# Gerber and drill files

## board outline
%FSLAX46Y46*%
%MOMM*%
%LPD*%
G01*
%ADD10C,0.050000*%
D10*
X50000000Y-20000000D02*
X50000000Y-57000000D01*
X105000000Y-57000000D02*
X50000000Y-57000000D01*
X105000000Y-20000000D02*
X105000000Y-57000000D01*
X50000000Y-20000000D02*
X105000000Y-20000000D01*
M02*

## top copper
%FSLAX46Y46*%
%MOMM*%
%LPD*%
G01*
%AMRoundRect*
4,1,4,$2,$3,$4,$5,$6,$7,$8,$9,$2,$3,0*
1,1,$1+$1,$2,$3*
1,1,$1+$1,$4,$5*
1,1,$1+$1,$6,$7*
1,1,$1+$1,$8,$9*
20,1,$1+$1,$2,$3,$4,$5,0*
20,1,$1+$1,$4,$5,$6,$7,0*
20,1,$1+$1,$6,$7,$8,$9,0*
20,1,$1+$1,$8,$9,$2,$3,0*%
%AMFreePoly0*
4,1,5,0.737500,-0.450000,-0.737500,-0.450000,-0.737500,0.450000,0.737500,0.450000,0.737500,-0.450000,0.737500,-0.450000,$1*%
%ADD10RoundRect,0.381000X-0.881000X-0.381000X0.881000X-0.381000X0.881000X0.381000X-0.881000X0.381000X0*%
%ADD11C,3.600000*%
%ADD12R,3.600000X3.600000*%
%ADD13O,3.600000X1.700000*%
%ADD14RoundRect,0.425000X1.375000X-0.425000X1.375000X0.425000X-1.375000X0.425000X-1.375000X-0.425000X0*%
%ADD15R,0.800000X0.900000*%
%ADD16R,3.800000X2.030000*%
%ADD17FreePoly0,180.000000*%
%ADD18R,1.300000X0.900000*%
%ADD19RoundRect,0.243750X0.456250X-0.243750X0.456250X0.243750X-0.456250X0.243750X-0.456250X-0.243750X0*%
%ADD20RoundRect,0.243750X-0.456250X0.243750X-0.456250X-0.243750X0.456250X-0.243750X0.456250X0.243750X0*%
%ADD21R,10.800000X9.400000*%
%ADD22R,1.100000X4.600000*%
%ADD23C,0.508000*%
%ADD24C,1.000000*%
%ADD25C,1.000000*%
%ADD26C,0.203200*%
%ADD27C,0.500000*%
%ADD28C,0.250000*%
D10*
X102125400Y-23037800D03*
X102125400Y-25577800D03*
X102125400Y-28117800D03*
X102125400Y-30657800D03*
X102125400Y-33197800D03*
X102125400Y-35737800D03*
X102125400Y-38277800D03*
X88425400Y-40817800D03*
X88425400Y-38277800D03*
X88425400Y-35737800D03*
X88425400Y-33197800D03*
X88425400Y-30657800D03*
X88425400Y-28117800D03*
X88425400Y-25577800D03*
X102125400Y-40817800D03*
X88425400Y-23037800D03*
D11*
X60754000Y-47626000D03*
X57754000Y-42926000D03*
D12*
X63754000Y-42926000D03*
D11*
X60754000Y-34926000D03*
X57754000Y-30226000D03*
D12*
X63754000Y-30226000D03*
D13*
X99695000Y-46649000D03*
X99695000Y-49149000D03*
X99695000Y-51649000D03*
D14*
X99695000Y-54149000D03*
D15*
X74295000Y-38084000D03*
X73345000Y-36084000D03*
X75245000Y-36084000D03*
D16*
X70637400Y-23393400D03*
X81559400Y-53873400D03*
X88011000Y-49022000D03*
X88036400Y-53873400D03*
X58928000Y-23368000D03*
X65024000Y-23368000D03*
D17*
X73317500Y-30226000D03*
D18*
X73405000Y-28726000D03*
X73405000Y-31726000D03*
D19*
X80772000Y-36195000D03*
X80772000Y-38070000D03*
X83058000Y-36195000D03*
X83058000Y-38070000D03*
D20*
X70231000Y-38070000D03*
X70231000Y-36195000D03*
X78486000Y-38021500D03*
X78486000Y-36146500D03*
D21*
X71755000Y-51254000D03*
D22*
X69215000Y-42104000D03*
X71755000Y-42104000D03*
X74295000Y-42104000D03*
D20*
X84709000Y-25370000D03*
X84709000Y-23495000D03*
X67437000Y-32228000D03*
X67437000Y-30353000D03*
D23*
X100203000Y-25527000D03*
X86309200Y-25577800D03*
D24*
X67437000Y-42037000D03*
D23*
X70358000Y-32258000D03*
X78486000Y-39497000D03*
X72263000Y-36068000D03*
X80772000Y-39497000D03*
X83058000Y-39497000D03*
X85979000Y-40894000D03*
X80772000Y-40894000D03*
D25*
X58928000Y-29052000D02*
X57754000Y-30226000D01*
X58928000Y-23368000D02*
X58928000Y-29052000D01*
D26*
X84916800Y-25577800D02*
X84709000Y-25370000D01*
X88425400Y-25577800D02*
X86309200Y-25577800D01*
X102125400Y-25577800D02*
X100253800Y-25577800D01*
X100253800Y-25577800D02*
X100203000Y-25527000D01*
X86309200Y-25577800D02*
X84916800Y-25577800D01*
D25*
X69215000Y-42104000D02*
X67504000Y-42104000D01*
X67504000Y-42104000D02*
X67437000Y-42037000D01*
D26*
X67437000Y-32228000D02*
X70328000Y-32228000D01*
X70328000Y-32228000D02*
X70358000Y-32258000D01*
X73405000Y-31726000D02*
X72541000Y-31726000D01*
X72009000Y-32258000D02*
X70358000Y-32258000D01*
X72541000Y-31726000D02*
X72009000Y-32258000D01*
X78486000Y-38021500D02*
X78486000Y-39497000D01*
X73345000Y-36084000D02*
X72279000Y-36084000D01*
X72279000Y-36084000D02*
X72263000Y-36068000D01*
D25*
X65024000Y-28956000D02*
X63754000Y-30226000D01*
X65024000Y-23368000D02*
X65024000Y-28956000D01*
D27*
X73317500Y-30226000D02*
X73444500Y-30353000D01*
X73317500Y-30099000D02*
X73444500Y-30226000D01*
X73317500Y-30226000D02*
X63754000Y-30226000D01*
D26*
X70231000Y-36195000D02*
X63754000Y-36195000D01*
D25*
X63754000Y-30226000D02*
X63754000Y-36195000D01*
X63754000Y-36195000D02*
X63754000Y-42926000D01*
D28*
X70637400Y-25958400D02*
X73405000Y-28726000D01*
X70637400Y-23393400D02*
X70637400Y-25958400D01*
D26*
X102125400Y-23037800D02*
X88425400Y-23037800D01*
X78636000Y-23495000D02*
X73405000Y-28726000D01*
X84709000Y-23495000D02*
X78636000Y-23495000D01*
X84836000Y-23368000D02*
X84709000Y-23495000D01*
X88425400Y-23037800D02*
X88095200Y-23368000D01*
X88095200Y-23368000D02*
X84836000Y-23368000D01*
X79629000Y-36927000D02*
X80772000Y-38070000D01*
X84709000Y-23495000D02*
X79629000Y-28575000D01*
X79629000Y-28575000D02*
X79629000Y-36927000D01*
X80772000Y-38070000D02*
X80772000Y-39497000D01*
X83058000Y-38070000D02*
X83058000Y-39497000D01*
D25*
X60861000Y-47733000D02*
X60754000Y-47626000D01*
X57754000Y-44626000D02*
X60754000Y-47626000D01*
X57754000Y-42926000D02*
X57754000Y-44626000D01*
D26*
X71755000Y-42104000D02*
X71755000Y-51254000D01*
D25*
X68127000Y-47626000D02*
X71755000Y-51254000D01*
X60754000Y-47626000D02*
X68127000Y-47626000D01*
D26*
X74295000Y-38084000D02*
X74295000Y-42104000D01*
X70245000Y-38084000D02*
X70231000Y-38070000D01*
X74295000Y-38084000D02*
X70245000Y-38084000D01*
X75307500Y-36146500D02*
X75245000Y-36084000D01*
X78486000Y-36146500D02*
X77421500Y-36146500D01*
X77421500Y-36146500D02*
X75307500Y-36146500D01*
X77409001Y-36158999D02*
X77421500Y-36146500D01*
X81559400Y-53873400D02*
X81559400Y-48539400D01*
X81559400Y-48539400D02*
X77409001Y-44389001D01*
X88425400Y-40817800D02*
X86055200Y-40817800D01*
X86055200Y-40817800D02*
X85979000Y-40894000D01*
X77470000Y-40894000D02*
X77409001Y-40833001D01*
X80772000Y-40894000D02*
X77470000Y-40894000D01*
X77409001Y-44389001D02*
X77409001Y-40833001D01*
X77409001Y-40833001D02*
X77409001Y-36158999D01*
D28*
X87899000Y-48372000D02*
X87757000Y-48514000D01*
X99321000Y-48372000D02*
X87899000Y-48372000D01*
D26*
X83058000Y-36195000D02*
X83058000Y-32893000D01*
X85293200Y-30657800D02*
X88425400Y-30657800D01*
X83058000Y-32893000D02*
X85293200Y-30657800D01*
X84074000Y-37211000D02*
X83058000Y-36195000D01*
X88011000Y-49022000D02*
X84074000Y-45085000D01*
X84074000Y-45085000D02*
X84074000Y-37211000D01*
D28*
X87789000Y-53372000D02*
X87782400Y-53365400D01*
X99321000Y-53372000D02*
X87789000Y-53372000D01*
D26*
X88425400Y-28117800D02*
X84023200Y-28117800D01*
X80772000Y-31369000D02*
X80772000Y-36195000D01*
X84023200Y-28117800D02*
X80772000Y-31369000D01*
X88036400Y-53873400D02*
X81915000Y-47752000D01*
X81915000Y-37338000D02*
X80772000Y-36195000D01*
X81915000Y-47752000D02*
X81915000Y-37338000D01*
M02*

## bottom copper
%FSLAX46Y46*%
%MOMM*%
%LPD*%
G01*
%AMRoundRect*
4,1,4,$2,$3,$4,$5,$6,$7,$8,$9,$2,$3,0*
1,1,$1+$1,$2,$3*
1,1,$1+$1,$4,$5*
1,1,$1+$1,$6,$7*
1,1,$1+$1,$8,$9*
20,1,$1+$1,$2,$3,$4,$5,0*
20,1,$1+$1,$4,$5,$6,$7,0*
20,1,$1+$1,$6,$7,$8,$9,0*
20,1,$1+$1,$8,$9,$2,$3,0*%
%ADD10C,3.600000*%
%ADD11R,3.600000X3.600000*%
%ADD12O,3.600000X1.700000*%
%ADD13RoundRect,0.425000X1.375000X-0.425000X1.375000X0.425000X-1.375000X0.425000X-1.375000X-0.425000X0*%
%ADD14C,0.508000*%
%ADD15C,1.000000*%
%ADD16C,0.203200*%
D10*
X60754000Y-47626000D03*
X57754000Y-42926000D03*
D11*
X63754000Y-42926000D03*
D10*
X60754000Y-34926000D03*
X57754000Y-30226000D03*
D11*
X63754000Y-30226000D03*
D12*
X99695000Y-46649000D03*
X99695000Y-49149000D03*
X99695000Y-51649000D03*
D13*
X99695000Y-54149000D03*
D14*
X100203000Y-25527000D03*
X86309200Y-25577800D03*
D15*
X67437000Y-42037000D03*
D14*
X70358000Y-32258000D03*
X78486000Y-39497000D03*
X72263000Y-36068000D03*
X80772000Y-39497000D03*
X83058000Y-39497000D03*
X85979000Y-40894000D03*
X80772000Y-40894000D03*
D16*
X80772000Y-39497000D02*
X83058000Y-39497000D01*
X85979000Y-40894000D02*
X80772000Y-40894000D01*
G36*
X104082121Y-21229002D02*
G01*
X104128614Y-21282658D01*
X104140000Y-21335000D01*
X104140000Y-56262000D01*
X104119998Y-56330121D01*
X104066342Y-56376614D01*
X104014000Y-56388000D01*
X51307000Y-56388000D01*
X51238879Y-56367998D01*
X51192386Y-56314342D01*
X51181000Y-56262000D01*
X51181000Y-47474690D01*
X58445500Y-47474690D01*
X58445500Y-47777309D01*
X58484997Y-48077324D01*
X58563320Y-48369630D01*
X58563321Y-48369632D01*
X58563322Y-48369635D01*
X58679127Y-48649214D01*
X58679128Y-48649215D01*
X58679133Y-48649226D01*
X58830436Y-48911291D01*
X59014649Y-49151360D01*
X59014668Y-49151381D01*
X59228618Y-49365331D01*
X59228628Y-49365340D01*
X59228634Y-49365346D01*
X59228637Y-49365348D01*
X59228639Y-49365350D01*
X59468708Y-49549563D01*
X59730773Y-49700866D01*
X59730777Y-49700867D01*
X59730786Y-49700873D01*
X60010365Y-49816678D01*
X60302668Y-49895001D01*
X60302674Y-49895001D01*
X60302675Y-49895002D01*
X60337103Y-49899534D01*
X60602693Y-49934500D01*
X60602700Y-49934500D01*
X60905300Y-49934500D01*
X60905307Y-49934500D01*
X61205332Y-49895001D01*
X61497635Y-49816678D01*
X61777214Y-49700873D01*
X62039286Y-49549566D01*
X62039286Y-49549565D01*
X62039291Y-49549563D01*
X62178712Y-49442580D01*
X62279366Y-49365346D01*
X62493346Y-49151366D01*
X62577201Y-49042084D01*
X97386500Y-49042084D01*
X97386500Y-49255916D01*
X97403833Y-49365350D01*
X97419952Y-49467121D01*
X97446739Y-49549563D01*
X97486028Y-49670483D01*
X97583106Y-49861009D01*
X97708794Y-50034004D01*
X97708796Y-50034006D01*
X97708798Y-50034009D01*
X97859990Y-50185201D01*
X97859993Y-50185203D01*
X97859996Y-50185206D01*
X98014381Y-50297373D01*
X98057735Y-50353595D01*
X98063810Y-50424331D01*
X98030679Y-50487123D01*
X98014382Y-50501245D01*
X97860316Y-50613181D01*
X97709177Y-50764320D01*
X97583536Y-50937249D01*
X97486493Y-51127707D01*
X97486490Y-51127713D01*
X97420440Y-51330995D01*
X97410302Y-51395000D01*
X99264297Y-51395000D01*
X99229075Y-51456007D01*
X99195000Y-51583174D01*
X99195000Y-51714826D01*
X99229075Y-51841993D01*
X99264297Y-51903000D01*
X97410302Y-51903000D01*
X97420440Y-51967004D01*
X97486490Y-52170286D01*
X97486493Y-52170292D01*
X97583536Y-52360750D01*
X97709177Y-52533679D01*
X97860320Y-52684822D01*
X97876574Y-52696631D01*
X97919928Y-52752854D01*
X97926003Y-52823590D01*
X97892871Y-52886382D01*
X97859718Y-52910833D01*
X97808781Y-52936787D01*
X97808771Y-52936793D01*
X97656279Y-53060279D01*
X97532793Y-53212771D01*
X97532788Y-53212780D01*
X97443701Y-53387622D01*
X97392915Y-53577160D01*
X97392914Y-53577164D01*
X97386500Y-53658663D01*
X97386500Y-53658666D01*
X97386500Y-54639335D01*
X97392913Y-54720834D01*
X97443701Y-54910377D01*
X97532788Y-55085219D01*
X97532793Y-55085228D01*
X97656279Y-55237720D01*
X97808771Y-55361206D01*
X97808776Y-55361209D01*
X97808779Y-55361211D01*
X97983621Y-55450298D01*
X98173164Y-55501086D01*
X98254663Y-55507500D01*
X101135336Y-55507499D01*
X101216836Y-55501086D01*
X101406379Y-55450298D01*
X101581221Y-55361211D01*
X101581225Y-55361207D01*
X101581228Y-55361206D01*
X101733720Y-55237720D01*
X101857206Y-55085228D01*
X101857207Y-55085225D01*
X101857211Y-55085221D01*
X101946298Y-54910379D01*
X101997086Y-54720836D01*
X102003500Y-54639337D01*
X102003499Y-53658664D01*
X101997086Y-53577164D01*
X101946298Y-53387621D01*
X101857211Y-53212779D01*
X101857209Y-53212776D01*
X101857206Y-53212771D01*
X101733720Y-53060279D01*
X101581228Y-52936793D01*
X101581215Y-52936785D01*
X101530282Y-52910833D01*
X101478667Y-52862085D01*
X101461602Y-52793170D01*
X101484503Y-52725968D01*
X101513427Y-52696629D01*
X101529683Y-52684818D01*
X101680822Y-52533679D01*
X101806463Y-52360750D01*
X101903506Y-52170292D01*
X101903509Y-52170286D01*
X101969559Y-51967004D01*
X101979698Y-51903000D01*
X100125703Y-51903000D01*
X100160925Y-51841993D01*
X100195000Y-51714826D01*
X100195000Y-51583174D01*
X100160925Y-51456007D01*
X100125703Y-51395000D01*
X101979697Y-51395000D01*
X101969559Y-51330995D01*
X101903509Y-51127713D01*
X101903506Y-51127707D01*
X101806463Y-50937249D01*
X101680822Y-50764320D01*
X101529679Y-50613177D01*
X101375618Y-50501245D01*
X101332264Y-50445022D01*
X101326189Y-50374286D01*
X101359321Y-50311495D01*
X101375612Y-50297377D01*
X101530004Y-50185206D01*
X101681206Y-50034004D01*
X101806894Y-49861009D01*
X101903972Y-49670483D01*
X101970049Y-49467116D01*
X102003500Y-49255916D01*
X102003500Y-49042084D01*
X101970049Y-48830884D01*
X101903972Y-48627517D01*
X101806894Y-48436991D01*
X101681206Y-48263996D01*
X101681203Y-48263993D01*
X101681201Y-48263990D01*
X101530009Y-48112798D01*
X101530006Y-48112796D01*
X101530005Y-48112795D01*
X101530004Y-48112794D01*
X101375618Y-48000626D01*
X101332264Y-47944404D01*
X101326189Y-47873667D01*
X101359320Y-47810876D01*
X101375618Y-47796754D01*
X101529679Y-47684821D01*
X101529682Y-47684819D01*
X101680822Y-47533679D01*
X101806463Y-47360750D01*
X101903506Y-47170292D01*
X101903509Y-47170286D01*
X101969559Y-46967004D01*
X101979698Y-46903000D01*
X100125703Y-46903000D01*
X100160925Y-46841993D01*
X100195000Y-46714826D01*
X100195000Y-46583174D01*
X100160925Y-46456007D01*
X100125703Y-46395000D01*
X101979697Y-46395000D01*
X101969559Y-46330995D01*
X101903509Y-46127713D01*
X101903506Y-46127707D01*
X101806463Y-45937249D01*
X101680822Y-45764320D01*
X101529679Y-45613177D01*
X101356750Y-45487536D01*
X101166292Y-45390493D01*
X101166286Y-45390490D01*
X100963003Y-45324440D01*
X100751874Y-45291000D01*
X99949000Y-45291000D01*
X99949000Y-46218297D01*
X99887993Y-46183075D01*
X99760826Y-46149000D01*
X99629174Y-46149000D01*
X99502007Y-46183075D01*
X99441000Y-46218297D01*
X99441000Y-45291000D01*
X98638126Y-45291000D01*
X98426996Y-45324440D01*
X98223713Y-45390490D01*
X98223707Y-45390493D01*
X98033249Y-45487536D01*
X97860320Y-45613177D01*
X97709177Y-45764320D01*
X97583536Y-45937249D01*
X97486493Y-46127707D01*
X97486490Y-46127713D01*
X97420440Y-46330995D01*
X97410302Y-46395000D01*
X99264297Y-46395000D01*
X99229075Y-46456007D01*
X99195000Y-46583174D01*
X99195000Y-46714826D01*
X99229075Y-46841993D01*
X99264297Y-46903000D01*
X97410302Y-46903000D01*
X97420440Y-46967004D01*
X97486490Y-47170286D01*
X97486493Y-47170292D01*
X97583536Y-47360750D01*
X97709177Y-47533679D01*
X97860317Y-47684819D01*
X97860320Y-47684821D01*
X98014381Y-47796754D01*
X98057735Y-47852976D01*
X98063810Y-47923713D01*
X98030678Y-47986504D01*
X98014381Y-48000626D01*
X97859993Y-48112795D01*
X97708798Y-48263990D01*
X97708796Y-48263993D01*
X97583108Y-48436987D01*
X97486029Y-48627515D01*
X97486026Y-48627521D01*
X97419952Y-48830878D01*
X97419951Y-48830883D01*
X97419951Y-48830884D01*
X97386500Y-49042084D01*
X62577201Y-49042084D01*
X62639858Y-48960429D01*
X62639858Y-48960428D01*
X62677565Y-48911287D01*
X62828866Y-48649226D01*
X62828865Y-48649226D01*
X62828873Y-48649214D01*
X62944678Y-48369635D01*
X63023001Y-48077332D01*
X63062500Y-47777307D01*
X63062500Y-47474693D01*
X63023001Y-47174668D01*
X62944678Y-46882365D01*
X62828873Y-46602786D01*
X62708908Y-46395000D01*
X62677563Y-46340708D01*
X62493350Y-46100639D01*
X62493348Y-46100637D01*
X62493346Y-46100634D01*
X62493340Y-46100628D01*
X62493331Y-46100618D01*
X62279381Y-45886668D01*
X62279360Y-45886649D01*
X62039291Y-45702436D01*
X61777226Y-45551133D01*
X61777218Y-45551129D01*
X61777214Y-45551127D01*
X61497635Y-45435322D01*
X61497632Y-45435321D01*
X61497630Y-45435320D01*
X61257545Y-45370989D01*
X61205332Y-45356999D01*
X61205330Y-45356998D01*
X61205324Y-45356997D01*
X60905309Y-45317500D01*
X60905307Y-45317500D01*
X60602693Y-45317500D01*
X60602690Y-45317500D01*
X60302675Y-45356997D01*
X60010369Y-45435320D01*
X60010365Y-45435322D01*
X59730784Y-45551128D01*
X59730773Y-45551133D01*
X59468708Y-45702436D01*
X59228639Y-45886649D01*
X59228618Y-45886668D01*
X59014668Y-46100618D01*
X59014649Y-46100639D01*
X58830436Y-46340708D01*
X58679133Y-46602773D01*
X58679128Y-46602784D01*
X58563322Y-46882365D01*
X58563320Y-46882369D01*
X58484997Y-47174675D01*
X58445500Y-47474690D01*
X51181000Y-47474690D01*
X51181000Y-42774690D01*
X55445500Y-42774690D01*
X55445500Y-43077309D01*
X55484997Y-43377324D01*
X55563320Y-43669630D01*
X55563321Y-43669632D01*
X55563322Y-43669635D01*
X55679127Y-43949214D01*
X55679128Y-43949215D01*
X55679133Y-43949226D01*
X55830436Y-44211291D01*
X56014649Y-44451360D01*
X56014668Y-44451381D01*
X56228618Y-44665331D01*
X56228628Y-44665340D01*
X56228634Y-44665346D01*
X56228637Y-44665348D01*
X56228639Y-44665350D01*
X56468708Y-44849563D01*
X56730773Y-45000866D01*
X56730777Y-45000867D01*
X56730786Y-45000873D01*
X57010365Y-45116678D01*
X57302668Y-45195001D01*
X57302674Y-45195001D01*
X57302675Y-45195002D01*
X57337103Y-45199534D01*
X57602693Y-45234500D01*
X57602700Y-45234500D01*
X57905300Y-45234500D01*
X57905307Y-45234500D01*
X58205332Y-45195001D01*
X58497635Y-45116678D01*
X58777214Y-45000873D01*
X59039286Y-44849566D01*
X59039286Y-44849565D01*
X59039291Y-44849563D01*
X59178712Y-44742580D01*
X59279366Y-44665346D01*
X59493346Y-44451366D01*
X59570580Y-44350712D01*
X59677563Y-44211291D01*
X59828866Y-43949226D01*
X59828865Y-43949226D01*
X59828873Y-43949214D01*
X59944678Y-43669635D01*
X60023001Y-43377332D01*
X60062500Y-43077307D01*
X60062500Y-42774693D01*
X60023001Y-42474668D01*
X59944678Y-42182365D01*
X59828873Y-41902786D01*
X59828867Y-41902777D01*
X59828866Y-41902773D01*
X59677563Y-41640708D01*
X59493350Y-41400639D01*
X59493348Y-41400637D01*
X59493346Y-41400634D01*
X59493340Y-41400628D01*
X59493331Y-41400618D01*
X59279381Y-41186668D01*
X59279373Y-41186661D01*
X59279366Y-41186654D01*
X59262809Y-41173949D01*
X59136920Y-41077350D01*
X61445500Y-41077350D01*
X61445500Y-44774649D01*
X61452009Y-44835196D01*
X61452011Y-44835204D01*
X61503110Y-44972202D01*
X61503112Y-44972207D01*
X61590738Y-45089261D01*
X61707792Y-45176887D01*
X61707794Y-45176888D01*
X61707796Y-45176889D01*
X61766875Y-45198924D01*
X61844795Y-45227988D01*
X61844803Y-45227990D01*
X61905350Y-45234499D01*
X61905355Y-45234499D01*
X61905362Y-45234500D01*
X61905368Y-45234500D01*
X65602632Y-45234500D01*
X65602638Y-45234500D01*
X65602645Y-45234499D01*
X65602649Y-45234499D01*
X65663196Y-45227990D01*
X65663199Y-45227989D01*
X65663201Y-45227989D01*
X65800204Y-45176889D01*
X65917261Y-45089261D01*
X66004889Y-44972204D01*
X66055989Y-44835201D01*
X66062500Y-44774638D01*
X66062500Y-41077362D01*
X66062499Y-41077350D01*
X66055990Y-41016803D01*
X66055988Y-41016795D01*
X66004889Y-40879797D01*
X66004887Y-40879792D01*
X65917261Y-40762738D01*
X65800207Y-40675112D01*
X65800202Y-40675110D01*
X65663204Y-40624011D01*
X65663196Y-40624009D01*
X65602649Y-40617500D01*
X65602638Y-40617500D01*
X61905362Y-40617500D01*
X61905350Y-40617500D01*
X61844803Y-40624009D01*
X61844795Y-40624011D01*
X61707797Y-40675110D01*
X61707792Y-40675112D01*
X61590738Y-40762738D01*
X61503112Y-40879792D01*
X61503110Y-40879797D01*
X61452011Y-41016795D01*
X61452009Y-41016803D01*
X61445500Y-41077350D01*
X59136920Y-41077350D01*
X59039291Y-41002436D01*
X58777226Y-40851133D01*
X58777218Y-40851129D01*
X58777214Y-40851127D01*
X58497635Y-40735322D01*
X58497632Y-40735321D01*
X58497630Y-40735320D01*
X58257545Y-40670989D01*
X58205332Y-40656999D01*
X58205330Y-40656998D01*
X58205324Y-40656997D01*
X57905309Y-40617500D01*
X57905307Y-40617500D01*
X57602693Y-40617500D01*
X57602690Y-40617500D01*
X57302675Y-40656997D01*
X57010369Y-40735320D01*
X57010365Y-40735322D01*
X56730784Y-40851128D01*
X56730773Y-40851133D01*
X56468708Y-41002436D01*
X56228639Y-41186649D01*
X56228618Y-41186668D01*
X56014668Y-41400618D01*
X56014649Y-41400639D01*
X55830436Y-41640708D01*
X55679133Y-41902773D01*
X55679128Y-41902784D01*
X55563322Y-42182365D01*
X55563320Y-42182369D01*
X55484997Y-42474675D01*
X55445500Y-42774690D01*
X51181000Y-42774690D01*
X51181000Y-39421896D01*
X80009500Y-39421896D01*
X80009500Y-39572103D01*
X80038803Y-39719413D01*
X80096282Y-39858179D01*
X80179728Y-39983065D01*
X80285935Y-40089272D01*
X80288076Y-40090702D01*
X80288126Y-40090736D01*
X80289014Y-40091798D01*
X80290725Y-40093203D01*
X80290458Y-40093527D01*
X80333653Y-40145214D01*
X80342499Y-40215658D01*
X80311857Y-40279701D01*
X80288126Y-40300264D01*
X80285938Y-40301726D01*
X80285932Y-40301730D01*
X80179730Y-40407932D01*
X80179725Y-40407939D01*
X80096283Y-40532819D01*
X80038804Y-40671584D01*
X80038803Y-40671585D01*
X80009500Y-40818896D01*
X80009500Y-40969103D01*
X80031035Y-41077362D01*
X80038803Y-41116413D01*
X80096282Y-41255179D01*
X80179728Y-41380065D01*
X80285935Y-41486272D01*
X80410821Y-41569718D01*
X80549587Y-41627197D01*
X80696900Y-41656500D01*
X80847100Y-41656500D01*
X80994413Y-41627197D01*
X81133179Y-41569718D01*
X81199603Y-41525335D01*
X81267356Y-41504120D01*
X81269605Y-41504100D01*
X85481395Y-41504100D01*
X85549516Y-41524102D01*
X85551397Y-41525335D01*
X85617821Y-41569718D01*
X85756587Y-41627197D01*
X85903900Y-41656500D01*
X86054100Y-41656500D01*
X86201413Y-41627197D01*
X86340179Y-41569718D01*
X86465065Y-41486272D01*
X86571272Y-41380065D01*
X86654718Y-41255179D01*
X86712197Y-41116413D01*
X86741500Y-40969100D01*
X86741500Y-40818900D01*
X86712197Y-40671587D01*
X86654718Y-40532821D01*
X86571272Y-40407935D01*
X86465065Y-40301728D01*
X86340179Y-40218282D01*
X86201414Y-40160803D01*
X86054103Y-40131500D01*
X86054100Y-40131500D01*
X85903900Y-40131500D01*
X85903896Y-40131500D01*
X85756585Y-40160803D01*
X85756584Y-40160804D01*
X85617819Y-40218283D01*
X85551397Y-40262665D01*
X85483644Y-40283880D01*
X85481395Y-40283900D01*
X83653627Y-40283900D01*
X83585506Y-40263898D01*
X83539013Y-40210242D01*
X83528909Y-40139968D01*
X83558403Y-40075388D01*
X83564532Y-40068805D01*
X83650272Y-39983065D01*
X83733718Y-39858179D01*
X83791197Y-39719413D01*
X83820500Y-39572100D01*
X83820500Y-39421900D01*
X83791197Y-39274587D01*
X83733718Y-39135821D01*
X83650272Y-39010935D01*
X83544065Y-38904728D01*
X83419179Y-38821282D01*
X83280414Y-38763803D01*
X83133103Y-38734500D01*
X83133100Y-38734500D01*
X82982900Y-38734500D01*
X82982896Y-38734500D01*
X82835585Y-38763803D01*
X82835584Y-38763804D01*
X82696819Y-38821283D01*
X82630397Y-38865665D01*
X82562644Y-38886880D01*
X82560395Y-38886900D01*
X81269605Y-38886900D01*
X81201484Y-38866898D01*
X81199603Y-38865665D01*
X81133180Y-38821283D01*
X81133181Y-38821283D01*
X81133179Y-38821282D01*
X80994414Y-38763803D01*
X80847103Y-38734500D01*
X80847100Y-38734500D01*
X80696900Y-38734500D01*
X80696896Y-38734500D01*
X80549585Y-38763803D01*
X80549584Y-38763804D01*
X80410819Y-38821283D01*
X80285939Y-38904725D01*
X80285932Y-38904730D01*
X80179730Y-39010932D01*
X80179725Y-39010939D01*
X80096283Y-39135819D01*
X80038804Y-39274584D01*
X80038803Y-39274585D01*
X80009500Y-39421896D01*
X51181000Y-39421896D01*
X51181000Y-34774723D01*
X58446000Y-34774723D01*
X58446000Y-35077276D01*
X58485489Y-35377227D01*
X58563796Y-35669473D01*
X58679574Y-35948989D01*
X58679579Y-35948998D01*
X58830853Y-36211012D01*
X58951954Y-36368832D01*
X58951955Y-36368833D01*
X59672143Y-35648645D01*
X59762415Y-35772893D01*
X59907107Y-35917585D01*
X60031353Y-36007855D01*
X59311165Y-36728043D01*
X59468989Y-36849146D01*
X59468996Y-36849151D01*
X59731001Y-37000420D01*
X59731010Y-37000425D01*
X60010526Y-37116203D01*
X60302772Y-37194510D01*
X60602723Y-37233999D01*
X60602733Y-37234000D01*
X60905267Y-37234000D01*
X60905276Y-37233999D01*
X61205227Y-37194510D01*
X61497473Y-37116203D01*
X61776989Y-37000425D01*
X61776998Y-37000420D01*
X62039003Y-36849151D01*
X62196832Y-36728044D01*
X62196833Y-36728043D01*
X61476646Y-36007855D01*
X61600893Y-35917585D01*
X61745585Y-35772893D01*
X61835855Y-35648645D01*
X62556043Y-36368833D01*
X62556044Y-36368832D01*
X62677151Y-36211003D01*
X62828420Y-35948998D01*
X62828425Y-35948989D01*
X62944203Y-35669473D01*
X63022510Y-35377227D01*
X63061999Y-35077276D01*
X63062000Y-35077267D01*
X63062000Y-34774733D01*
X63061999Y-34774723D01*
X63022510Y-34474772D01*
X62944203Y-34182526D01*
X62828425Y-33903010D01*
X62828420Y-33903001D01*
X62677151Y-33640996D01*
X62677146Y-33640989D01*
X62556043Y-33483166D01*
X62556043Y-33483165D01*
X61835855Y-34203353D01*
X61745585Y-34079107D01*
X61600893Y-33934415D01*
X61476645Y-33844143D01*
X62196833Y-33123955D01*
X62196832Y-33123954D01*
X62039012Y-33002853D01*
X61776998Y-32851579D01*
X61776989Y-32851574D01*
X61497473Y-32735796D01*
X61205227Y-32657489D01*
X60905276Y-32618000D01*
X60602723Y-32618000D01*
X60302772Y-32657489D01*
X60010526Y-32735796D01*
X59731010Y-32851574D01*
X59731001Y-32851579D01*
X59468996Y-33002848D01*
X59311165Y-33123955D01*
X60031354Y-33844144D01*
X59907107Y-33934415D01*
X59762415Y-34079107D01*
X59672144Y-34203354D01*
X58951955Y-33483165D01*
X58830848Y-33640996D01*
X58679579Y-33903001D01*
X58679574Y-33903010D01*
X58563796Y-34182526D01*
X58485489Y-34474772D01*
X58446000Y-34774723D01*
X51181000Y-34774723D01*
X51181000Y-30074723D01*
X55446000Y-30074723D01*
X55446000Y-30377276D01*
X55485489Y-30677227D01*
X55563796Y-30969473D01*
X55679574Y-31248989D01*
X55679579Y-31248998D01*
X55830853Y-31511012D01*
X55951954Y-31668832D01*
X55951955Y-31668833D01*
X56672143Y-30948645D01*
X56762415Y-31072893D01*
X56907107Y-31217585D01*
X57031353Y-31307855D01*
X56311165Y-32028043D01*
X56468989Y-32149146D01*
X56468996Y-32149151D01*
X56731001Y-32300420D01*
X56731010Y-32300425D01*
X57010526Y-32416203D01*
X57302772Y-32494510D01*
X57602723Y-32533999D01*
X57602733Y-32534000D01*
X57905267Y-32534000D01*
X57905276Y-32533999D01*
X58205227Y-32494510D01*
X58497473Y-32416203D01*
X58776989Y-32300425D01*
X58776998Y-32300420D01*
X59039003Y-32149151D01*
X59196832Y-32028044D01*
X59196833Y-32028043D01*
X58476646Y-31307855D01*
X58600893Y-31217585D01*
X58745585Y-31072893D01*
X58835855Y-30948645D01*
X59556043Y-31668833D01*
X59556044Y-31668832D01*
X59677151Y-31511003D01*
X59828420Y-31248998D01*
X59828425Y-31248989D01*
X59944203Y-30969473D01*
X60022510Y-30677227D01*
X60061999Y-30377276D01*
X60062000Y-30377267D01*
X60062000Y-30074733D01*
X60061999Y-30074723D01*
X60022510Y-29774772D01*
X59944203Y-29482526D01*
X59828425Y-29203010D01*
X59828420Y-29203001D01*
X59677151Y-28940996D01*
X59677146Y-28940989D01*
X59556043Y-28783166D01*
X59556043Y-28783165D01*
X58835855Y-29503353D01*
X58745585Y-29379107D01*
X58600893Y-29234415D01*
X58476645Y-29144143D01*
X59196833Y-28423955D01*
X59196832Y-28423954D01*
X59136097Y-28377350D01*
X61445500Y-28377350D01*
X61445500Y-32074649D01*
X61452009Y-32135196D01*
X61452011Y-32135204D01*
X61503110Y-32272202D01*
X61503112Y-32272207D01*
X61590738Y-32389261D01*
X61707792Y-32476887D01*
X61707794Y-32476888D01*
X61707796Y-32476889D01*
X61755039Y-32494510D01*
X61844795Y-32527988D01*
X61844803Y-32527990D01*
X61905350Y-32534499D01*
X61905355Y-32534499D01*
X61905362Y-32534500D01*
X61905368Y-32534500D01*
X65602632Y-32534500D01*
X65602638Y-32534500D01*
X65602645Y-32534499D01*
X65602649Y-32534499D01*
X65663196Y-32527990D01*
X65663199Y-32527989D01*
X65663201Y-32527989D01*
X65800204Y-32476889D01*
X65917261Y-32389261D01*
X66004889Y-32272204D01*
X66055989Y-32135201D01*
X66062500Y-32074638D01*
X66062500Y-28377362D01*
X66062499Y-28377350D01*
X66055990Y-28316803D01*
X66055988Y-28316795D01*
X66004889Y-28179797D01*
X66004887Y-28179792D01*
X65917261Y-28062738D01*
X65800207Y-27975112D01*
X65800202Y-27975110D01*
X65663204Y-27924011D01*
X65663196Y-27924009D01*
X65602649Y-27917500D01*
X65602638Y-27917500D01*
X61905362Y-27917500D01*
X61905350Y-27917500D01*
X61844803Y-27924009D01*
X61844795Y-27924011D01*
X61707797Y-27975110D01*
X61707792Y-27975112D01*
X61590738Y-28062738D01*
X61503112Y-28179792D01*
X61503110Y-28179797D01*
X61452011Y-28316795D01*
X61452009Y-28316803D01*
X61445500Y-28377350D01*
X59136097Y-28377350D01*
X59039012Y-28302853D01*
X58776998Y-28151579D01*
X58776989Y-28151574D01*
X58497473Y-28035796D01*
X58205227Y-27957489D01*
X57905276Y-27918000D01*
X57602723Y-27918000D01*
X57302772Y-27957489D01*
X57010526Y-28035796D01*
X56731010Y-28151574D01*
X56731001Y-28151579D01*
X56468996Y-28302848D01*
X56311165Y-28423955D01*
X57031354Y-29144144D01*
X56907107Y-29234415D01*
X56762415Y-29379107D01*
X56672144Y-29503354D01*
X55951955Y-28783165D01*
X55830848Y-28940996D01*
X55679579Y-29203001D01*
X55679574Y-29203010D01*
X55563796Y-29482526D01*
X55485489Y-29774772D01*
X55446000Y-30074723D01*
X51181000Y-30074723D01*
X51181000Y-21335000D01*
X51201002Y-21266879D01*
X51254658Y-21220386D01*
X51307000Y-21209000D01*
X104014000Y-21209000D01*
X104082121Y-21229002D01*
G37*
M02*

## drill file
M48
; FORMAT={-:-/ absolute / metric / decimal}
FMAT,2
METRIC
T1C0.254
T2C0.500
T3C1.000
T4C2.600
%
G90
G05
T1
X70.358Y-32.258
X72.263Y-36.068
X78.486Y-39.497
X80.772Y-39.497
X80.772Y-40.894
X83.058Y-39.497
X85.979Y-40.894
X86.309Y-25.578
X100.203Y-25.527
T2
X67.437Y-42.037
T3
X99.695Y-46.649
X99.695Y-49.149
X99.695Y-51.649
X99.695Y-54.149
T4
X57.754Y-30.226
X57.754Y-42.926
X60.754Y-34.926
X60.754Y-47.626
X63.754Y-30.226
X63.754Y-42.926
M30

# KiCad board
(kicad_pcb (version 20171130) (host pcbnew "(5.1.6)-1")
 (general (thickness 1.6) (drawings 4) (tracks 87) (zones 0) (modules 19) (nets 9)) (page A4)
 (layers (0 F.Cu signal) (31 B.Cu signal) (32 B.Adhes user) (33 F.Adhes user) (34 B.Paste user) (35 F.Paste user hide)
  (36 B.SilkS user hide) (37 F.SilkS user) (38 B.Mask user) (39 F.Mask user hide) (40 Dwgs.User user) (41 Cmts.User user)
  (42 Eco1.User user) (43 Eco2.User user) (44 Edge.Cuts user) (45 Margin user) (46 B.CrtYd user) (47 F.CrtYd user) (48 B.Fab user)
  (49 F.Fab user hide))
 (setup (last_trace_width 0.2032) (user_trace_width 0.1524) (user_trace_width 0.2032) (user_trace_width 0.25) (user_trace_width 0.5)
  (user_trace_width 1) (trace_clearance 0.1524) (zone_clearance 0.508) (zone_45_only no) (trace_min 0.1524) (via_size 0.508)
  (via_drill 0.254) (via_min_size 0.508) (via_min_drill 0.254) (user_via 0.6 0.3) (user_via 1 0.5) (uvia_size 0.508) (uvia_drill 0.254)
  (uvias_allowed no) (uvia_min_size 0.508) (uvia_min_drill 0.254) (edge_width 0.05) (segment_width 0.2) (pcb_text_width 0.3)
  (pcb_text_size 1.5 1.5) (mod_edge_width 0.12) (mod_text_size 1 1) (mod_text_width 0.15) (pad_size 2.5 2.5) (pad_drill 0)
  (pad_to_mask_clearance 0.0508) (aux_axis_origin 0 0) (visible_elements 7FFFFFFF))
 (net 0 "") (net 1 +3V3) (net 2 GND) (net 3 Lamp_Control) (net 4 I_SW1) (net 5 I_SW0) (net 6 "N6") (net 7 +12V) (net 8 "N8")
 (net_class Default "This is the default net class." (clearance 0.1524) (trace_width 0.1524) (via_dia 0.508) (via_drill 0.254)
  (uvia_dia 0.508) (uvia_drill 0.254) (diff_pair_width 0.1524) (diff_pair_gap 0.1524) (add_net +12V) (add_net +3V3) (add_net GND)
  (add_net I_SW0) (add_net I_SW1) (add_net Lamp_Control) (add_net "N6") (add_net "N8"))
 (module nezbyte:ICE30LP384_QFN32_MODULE (layer F.Cu) (at 95.25 31.75)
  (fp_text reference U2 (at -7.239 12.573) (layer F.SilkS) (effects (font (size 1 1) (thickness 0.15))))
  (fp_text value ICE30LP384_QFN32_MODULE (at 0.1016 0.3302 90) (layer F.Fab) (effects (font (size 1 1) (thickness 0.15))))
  (pad 16 smd roundrect (at 6.8754 -8.7122) (size 2.524 1.524) (layers F.Cu F.Paste F.Mask) (roundrect_rratio 0.25) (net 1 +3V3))
  (pad 15 smd roundrect (at 6.8754 -6.1722) (size 2.524 1.524) (layers F.Cu F.Paste F.Mask) (roundrect_rratio 0.25) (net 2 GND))
  (pad 14 smd roundrect (at 6.8754 -3.6322) (size 2.524 1.524) (layers F.Cu F.Paste F.Mask) (roundrect_rratio 0.25))
  (pad 13 smd roundrect (at 6.8754 -1.0922) (size 2.524 1.524) (layers F.Cu F.Paste F.Mask) (roundrect_rratio 0.25))
  (pad 12 smd roundrect (at 6.8754 1.4478) (size 2.524 1.524) (layers F.Cu F.Paste F.Mask) (roundrect_rratio 0.25))
  (pad 11 smd roundrect (at 6.8754 3.9878) (size 2.524 1.524) (layers F.Cu F.Paste F.Mask) (roundrect_rratio 0.25))
  (pad 10 smd roundrect (at 6.8754 6.5278) (size 2.524 1.524) (layers F.Cu F.Paste F.Mask) (roundrect_rratio 0.25))
  (pad 8 smd roundrect (at -6.8246 9.0678) (size 2.524 1.524) (layers F.Cu F.Paste F.Mask) (roundrect_rratio 0.25) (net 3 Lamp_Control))
  (pad 7 smd roundrect (at -6.8246 6.5278) (size 2.524 1.524) (layers F.Cu F.Paste F.Mask) (roundrect_rratio 0.25))
  (pad 6 smd roundrect (at -6.8246 3.9878) (size 2.524 1.524) (layers F.Cu F.Paste F.Mask) (roundrect_rratio 0.25))
  (pad 5 smd roundrect (at -6.8246 1.4478) (size 2.524 1.524) (layers F.Cu F.Paste F.Mask) (roundrect_rratio 0.25))
  (pad 4 smd roundrect (at -6.8246 -1.0922) (size 2.524 1.524) (layers F.Cu F.Paste F.Mask) (roundrect_rratio 0.25) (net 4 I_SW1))
  (pad 3 smd roundrect (at -6.8246 -3.6322) (size 2.524 1.524) (layers F.Cu F.Paste F.Mask) (roundrect_rratio 0.25) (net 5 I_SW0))
  (pad 2 smd roundrect (at -6.8246 -6.1722) (size 2.524 1.524) (layers F.Cu F.Paste F.Mask) (roundrect_rratio 0.25) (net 2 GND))
  (pad 9 smd roundrect (at 6.8754 9.0678) (size 2.524 1.524) (layers F.Cu F.Paste F.Mask) (roundrect_rratio 0.25))
  (pad 1 smd roundrect (at -6.8246 -8.7122) (size 2.524 1.524) (layers F.Cu F.Paste F.Mask) (roundrect_rratio 0.25) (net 1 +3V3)))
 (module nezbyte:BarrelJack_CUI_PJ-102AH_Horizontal (layer F.Cu) (at 63.754 42.926 270)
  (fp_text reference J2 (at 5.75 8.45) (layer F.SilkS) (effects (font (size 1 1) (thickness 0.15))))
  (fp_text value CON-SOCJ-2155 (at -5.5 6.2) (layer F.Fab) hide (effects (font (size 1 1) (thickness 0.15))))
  (pad 3 thru_hole circle (at 4.7 3 270) (size 3.6 3.6) (drill 2.6) (layers *.Cu *.Mask) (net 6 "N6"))
  (pad 2 thru_hole circle (at 0 6 270) (size 3.6 3.6) (drill 2.6) (layers *.Cu *.Mask) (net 6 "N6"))
  (pad 1 thru_hole rect (at 0 0 270) (size 3.6 3.6) (drill 2.6) (layers *.Cu *.Mask) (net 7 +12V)))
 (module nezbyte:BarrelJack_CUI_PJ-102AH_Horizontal (layer F.Cu) (at 63.754 30.226 270)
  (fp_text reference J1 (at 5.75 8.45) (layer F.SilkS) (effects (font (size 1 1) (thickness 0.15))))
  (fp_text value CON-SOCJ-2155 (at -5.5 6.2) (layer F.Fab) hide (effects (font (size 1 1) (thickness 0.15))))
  (pad 3 thru_hole circle (at 4.7 3 270) (size 3.6 3.6) (drill 2.6) (layers *.Cu *.Mask) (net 2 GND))
  (pad 2 thru_hole circle (at 0 6 270) (size 3.6 3.6) (drill 2.6) (layers *.Cu *.Mask) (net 2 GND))
  (pad 1 thru_hole rect (at 0 0 270) (size 3.6 3.6) (drill 2.6) (layers *.Cu *.Mask) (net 7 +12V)))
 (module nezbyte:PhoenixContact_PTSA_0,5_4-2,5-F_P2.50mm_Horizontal (layer F.Cu) (at 92.195 56.149 90)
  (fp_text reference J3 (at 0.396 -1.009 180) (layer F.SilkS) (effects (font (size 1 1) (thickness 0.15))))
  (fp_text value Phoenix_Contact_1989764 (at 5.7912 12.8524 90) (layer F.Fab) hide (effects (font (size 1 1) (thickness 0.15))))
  (pad 4 thru_hole oval (at 9.5 7.5 90) (size 1.7 3.6) (drill 1) (layers *.Cu *.Mask) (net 2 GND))
  (pad 3 thru_hole oval (at 7 7.5 90) (size 1.7 3.6) (drill 1) (layers *.Cu *.Mask) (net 4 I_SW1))
  (pad 2 thru_hole oval (at 4.5 7.5 90) (size 1.7 3.6) (drill 1) (layers *.Cu *.Mask) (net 2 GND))
  (pad 1 thru_hole roundrect (at 2 7.5 90) (size 1.7 3.6) (drill 1) (layers *.Cu *.Mask) (roundrect_rratio 0.25) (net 5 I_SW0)))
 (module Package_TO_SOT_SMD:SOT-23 (layer F.Cu) (at 74.295 37.084 270)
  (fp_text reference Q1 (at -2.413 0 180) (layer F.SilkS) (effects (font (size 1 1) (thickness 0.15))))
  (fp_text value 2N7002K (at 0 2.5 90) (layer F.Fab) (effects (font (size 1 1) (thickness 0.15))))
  (pad 3 smd rect (at 1 0 270) (size 0.9 0.8) (layers F.Cu F.Paste F.Mask) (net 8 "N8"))
  (pad 2 smd rect (at -1 0.95 270) (size 0.9 0.8) (layers F.Cu F.Paste F.Mask) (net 2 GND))
  (pad 1 smd rect (at -1 -0.95 270) (size 0.9 0.8) (layers F.Cu F.Paste F.Mask) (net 3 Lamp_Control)))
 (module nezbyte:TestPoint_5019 (layer F.Cu) (at 70.612 23.368)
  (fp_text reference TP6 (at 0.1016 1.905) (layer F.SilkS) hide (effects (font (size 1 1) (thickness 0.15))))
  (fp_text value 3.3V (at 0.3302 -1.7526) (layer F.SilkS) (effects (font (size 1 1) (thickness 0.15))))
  (pad 1 smd rect (at 0.0254 0.0254) (size 3.8 2.03) (layers F.Cu F.Paste F.Mask) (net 1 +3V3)))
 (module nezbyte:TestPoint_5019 (layer F.Cu) (at 81.534 53.848)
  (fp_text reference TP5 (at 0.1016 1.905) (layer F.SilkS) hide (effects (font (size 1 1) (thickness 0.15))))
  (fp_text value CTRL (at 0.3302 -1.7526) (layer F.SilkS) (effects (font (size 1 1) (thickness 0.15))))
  (pad 1 smd rect (at 0.0254 0.0254) (size 3.8 2.03) (layers F.Cu F.Paste F.Mask) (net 3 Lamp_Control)))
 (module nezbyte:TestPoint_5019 (layer F.Cu) (at 87.9856 48.9966)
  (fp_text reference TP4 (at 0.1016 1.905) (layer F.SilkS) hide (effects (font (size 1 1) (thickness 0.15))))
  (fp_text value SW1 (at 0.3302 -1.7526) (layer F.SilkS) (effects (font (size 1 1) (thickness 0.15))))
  (pad 1 smd rect (at 0.0254 0.0254) (size 3.8 2.03) (layers F.Cu F.Paste F.Mask) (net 4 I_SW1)))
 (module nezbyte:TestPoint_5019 (layer F.Cu) (at 88.011 53.848)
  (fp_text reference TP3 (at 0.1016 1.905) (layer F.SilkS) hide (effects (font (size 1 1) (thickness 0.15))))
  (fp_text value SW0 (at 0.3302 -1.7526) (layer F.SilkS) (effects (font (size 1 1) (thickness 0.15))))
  (pad 1 smd rect (at 0.0254 0.0254) (size 3.8 2.03) (layers F.Cu F.Paste F.Mask) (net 5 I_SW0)))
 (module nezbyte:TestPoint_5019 (layer F.Cu) (at 58.9026 23.3426)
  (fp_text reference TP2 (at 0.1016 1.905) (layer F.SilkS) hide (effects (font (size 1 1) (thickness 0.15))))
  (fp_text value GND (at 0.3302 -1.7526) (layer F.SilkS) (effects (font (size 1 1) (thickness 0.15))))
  (pad 1 smd rect (at 0.0254 0.0254) (size 3.8 2.03) (layers F.Cu F.Paste F.Mask) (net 2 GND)))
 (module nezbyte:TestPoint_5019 (layer F.Cu) (at 64.9986 23.3426)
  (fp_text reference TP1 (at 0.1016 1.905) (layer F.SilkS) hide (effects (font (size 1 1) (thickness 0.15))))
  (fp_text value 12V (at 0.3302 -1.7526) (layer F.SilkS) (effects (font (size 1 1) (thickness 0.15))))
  (pad 1 smd rect (at 0.0254 0.0254) (size 3.8 2.03) (layers F.Cu F.Paste F.Mask) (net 7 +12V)))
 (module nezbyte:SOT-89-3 (layer F.Cu) (at 71.755 30.226 180)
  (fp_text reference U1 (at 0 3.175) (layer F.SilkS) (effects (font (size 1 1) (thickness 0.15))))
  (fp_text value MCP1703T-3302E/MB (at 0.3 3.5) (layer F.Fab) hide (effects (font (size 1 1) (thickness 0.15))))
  (pad 2 smd custom (at -1.5625 0 180) (size 1.475 0.9) (layers F.Cu F.Paste F.Mask) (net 7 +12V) (zone_connect 2)
   (options (clearance outline) (anchor rect)) (primitives))
  (pad 3 smd rect (at -1.65 1.5 180) (size 1.3 0.9) (layers F.Cu F.Paste F.Mask) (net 1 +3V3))
  (pad 1 smd rect (at -1.65 -1.5 180) (size 1.3 0.9) (layers F.Cu F.Paste F.Mask) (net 2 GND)))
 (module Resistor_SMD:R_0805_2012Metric (layer F.Cu) (at 80.772 37.1325 90)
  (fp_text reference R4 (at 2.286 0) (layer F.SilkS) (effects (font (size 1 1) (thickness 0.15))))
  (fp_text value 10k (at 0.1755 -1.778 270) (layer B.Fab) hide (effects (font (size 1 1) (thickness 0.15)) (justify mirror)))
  (pad 2 smd roundrect (at 0.9375 0 90) (size 0.975 1.4) (layers F.Cu F.Paste F.Mask) (roundrect_rratio 0.25) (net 5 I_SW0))
  (pad 1 smd roundrect (at -0.9375 0 90) (size 0.975 1.4) (layers F.Cu F.Paste F.Mask) (roundrect_rratio 0.25) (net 1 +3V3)))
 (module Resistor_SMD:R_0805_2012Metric (layer F.Cu) (at 83.058 37.1325 90)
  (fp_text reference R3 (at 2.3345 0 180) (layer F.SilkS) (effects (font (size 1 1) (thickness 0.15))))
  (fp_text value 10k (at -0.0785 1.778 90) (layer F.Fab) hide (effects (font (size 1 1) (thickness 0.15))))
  (pad 2 smd roundrect (at 0.9375 0 90) (size 0.975 1.4) (layers F.Cu F.Paste F.Mask) (roundrect_rratio 0.25) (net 4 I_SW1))
  (pad 1 smd roundrect (at -0.9375 0 90) (size 0.975 1.4) (layers F.Cu F.Paste F.Mask) (roundrect_rratio 0.25) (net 1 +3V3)))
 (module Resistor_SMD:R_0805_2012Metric (layer F.Cu) (at 70.231 37.1325 270)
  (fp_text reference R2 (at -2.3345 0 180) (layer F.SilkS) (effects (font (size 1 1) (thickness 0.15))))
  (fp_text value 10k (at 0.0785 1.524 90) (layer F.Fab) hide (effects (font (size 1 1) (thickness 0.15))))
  (pad 2 smd roundrect (at 0.9375 0 270) (size 0.975 1.4) (layers F.Cu F.Paste F.Mask) (roundrect_rratio 0.25) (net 8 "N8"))
  (pad 1 smd roundrect (at -0.9375 0 270) (size 0.975 1.4) (layers F.Cu F.Paste F.Mask) (roundrect_rratio 0.25) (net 7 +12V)))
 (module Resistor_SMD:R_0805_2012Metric (layer F.Cu) (at 78.486 37.084 270)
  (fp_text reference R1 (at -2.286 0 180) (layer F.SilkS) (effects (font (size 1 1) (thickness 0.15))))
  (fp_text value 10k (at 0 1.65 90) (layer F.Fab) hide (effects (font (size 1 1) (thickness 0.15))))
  (pad 2 smd roundrect (at 0.9375 0 270) (size 0.975 1.4) (layers F.Cu F.Paste F.Mask) (roundrect_rratio 0.25) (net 2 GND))
  (pad 1 smd roundrect (at -0.9375 0 270) (size 0.975 1.4) (layers F.Cu F.Paste F.Mask) (roundrect_rratio 0.25) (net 3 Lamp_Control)))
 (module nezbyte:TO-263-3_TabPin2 (layer F.Cu) (at 71.755 47.879 270)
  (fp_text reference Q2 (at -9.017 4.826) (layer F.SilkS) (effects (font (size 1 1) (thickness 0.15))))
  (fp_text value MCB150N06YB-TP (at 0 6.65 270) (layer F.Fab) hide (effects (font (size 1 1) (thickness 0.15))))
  (pad "" smd rect (at 0.95 2.775 270) (size 4.55 5.25) (layers F.Paste))
  (pad "" smd rect (at 5.8 -2.775 270) (size 4.55 5.25) (layers F.Paste))
  (pad "" smd rect (at 0.95 -2.775 270) (size 4.55 5.25) (layers F.Paste))
  (pad "" smd rect (at 5.8 2.775 270) (size 4.55 5.25) (layers F.Paste))
  (pad 2 smd rect (at 3.375 0 270) (size 9.4 10.8) (layers F.Cu F.Mask) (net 6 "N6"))
  (pad 3 smd rect (at -5.775 2.54 270) (size 4.6 1.1) (layers F.Cu F.Paste F.Mask) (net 2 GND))
  (pad 2 smd rect (at -5.775 0 270) (size 4.6 1.1) (layers F.Cu F.Paste F.Mask) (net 6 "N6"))
  (pad 1 smd rect (at -5.775 -2.54 270) (size 4.6 1.1) (layers F.Cu F.Paste F.Mask) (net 8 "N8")))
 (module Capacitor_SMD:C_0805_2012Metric (layer F.Cu) (at 84.709 24.4325 270)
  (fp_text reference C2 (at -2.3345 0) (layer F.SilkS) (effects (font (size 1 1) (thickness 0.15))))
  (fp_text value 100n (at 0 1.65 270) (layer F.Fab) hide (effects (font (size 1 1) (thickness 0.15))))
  (pad 2 smd roundrect (at 0.9375 0 270) (size 0.975 1.4) (layers F.Cu F.Paste F.Mask) (roundrect_rratio 0.25) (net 2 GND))
  (pad 1 smd roundrect (at -0.9375 0 270) (size 0.975 1.4) (layers F.Cu F.Paste F.Mask) (roundrect_rratio 0.25) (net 1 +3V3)))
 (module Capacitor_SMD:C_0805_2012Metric (layer F.Cu) (at 67.437 31.2905 270)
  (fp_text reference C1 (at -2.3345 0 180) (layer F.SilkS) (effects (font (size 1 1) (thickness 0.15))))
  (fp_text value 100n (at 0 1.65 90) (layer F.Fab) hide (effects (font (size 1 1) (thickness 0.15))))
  (pad 2 smd roundrect (at 0.9375 0 270) (size 0.975 1.4) (layers F.Cu F.Paste F.Mask) (roundrect_rratio 0.25) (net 2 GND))
  (pad 1 smd roundrect (at -0.9375 0 270) (size 0.975 1.4) (layers F.Cu F.Paste F.Mask) (roundrect_rratio 0.25) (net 7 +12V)))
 (gr_line (start 50 20) (end 50 57) (layer Edge.Cuts) (width 0.05))
 (gr_line (start 105 57) (end 50 57) (layer Edge.Cuts) (width 0.05))
 (gr_line (start 105 20) (end 105 57) (layer Edge.Cuts) (width 0.05))
 (gr_line (start 50 20) (end 105 20) (layer Edge.Cuts) (width 0.05))
 (segment (start 58.928 29.052) (end 57.754 30.226) (width 1) (layer F.Cu) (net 2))
 (segment (start 58.928 23.368) (end 58.928 29.052) (width 1) (layer F.Cu) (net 2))
 (segment (start 84.9168 25.5778) (end 84.709 25.37) (width 0.2032) (layer F.Cu) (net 2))
 (segment (start 88.4254 25.5778) (end 86.3092 25.5778) (width 0.2032) (layer F.Cu) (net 2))
 (via (at 100.203 25.527) (size 0.508) (drill 0.254) (layers F.Cu B.Cu) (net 2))
 (segment (start 102.1254 25.5778) (end 100.2538 25.5778) (width 0.2032) (layer F.Cu) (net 2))
 (segment (start 100.2538 25.5778) (end 100.203 25.527) (width 0.2032) (layer F.Cu) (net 2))
 (segment (start 86.3092 25.5778) (end 84.9168 25.5778) (width 0.2032) (layer F.Cu) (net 2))
 (via (at 86.3092 25.5778) (size 0.508) (drill 0.254) (layers F.Cu B.Cu) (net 2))
 (via (at 67.437 42.037) (size 1) (drill 0.5) (layers F.Cu B.Cu) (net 2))
 (segment (start 69.215 42.104) (end 67.504 42.104) (width 1) (layer F.Cu) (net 2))
 (segment (start 67.504 42.104) (end 67.437 42.037) (width 1) (layer F.Cu) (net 2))
 (segment (start 67.437 32.228) (end 70.328 32.228) (width 0.2032) (layer F.Cu) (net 2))
 (via (at 70.358 32.258) (size 0.508) (drill 0.254) (layers F.Cu B.Cu) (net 2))
 (segment (start 70.328 32.228) (end 70.358 32.258) (width 0.2032) (layer F.Cu) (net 2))
 (segment (start 73.405 31.726) (end 72.541 31.726) (width 0.2032) (layer F.Cu) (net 2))
 (segment (start 72.009 32.258) (end 70.358 32.258) (width 0.2032) (layer F.Cu) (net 2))
 (segment (start 72.541 31.726) (end 72.009 32.258) (width 0.2032) (layer F.Cu) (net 2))
 (via (at 78.486 39.497) (size 0.508) (drill 0.254) (layers F.Cu B.Cu) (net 2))
 (segment (start 78.486 38.0215) (end 78.486 39.497) (width 0.2032) (layer F.Cu) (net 2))
 (via (at 72.263 36.068) (size 0.508) (drill 0.254) (layers F.Cu B.Cu) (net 2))
 (segment (start 73.345 36.084) (end 72.279 36.084) (width 0.2032) (layer F.Cu) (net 2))
 (segment (start 72.279 36.084) (end 72.263 36.068) (width 0.2032) (layer F.Cu) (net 2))
 (segment (start 65.024 28.956) (end 63.754 30.226) (width 1) (layer F.Cu) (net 7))
 (segment (start 65.024 23.368) (end 65.024 28.956) (width 1) (layer F.Cu) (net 7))
 (segment (start 73.3175 30.226) (end 73.4445 30.353) (width 0.5) (layer F.Cu) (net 7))
 (segment (start 73.3175 30.099) (end 73.4445 30.226) (width 0.5) (layer F.Cu) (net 7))
 (segment (start 73.3175 30.226) (end 63.754 30.226) (width 0.5) (layer F.Cu) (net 7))
 (segment (start 70.231 36.195) (end 63.754 36.195) (width 0.2032) (layer F.Cu) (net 7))
 (segment (start 63.754 30.226) (end 63.754 36.195) (width 1) (layer F.Cu) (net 7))
 (segment (start 63.754 36.195) (end 63.754 42.926) (width 1) (layer F.Cu) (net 7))
 (segment (start 70.6374 25.9584) (end 73.405 28.726) (width 0.25) (layer F.Cu) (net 1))
 (segment (start 70.6374 23.3934) (end 70.6374 25.9584) (width 0.25) (layer F.Cu) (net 1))
 (segment (start 102.1254 23.0378) (end 88.4254 23.0378) (width 0.2032) (layer F.Cu) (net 1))
 (segment (start 78.636 23.495) (end 73.405 28.726) (width 0.2032) (layer F.Cu) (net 1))
 (segment (start 84.709 23.495) (end 78.636 23.495) (width 0.2032) (layer F.Cu) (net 1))
 (segment (start 84.836 23.368) (end 84.709 23.495) (width 0.2032) (layer F.Cu) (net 1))
 (segment (start 88.4254 23.0378) (end 88.0952 23.368) (width 0.2032) (layer F.Cu) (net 1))
 (segment (start 88.0952 23.368) (end 84.836 23.368) (width 0.2032) (layer F.Cu) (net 1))
 (segment (start 79.629 36.927) (end 80.772 38.07) (width 0.2032) (layer F.Cu) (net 1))
 (segment (start 84.709 23.495) (end 79.629 28.575) (width 0.2032) (layer F.Cu) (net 1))
 (segment (start 79.629 28.575) (end 79.629 36.927) (width 0.2032) (layer F.Cu) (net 1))
 (via (at 80.772 39.497) (size 0.508) (drill 0.254) (layers F.Cu B.Cu) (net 1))
 (segment (start 80.772 38.07) (end 80.772 39.497) (width 0.2032) (layer F.Cu) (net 1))
 (segment (start 80.772 39.497) (end 83.058 39.497) (width 0.2032) (layer B.Cu) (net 1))
 (via (at 83.058 39.497) (size 0.508) (drill 0.254) (layers F.Cu B.Cu) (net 1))
 (segment (start 83.058 38.07) (end 83.058 39.497) (width 0.2032) (layer F.Cu) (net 1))
 (segment (start 60.861 47.733) (end 60.754 47.626) (width 1) (layer F.Cu) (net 6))
 (segment (start 57.754 44.626) (end 60.754 47.626) (width 1) (layer F.Cu) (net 6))
 (segment (start 57.754 42.926) (end 57.754 44.626) (width 1) (layer F.Cu) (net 6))
 (segment (start 71.755 42.104) (end 71.755 51.254) (width 0.2032) (layer F.Cu) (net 6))
 (segment (start 68.127 47.626) (end 71.755 51.254) (width 1) (layer F.Cu) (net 6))
 (segment (start 60.754 47.626) (end 68.127 47.626) (width 1) (layer F.Cu) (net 6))
 (segment (start 74.295 38.084) (end 74.295 42.104) (width 0.2032) (layer F.Cu) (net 8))
 (segment (start 70.245 38.084) (end 70.231 38.07) (width 0.2032) (layer F.Cu) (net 8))
 (segment (start 74.295 38.084) (end 70.245 38.084) (width 0.2032) (layer F.Cu) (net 8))
 (segment (start 75.3075 36.1465) (end 75.245 36.084) (width 0.2032) (layer F.Cu) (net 3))
 (segment (start 78.486 36.1465) (end 77.4215 36.1465) (width 0.2032) (layer F.Cu) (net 3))
 (segment (start 77.4215 36.1465) (end 75.3075 36.1465) (width 0.2032) (layer F.Cu) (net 3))
 (segment (start 77.409001 36.158999) (end 77.4215 36.1465) (width 0.2032) (layer F.Cu) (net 3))
 (segment (start 81.5594 53.8734) (end 81.5594 48.5394) (width 0.2032) (layer F.Cu) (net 3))
 (segment (start 81.5594 48.5394) (end 77.409001 44.389001) (width 0.2032) (layer F.Cu) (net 3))
 (via (at 85.979 40.894) (size 0.508) (drill 0.254) (layers F.Cu B.Cu) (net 3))
 (segment (start 88.4254 40.8178) (end 86.0552 40.8178) (width 0.2032) (layer F.Cu) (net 3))
 (segment (start 86.0552 40.8178) (end 85.979 40.894) (width 0.2032) (layer F.Cu) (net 3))
 (via (at 80.772 40.894) (size 0.508) (drill 0.254) (layers F.Cu B.Cu) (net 3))
 (segment (start 85.979 40.894) (end 80.772 40.894) (width 0.2032) (layer B.Cu) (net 3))
 (segment (start 77.47 40.894) (end 77.409001 40.833001) (width 0.2032) (layer F.Cu) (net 3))
 (segment (start 80.772 40.894) (end 77.47 40.894) (width 0.2032) (layer F.Cu) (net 3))
 (segment (start 77.409001 44.389001) (end 77.409001 40.833001) (width 0.2032) (layer F.Cu) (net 3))
 (segment (start 77.409001 40.833001) (end 77.409001 36.158999) (width 0.2032) (layer F.Cu) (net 3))
 (segment (start 87.899 48.372) (end 87.757 48.514) (width 0.25) (layer F.Cu) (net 4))
 (segment (start 99.321 48.372) (end 87.899 48.372) (width 0.25) (layer F.Cu) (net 4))
 (segment (start 83.058 36.195) (end 83.058 32.893) (width 0.2032) (layer F.Cu) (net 4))
 (segment (start 85.2932 30.6578) (end 88.4254 30.6578) (width 0.2032) (layer F.Cu) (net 4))
 (segment (start 83.058 32.893) (end 85.2932 30.6578) (width 0.2032) (layer F.Cu) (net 4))
 (segment (start 84.074 37.211) (end 83.058 36.195) (width 0.2032) (layer F.Cu) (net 4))
 (segment (start 88.011 49.022) (end 84.074 45.085) (width 0.2032) (layer F.Cu) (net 4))
 (segment (start 84.074 45.085) (end 84.074 37.211) (width 0.2032) (layer F.Cu) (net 4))
 (segment (start 87.789 53.372) (end 87.7824 53.3654) (width 0.25) (layer F.Cu) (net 5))
 (segment (start 99.321 53.372) (end 87.789 53.372) (width 0.25) (layer F.Cu) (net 5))
 (segment (start 88.4254 28.1178) (end 84.0232 28.1178) (width 0.2032) (layer F.Cu) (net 5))
 (segment (start 80.772 31.369) (end 80.772 36.195) (width 0.2032) (layer F.Cu) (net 5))
 (segment (start 84.0232 28.1178) (end 80.772 31.369) (width 0.2032) (layer F.Cu) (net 5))
 (segment (start 88.0364 53.8734) (end 81.915 47.752) (width 0.2032) (layer F.Cu) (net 5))
 (segment (start 81.915 37.338) (end 80.772 36.195) (width 0.2032) (layer F.Cu) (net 5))
 (segment (start 81.915 47.752) (end 81.915 37.338) (width 0.2032) (layer F.Cu) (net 5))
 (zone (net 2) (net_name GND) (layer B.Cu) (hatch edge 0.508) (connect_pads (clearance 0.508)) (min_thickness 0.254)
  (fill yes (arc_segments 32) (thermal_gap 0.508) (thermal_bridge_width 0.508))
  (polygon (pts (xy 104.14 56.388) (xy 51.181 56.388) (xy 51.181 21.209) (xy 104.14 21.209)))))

